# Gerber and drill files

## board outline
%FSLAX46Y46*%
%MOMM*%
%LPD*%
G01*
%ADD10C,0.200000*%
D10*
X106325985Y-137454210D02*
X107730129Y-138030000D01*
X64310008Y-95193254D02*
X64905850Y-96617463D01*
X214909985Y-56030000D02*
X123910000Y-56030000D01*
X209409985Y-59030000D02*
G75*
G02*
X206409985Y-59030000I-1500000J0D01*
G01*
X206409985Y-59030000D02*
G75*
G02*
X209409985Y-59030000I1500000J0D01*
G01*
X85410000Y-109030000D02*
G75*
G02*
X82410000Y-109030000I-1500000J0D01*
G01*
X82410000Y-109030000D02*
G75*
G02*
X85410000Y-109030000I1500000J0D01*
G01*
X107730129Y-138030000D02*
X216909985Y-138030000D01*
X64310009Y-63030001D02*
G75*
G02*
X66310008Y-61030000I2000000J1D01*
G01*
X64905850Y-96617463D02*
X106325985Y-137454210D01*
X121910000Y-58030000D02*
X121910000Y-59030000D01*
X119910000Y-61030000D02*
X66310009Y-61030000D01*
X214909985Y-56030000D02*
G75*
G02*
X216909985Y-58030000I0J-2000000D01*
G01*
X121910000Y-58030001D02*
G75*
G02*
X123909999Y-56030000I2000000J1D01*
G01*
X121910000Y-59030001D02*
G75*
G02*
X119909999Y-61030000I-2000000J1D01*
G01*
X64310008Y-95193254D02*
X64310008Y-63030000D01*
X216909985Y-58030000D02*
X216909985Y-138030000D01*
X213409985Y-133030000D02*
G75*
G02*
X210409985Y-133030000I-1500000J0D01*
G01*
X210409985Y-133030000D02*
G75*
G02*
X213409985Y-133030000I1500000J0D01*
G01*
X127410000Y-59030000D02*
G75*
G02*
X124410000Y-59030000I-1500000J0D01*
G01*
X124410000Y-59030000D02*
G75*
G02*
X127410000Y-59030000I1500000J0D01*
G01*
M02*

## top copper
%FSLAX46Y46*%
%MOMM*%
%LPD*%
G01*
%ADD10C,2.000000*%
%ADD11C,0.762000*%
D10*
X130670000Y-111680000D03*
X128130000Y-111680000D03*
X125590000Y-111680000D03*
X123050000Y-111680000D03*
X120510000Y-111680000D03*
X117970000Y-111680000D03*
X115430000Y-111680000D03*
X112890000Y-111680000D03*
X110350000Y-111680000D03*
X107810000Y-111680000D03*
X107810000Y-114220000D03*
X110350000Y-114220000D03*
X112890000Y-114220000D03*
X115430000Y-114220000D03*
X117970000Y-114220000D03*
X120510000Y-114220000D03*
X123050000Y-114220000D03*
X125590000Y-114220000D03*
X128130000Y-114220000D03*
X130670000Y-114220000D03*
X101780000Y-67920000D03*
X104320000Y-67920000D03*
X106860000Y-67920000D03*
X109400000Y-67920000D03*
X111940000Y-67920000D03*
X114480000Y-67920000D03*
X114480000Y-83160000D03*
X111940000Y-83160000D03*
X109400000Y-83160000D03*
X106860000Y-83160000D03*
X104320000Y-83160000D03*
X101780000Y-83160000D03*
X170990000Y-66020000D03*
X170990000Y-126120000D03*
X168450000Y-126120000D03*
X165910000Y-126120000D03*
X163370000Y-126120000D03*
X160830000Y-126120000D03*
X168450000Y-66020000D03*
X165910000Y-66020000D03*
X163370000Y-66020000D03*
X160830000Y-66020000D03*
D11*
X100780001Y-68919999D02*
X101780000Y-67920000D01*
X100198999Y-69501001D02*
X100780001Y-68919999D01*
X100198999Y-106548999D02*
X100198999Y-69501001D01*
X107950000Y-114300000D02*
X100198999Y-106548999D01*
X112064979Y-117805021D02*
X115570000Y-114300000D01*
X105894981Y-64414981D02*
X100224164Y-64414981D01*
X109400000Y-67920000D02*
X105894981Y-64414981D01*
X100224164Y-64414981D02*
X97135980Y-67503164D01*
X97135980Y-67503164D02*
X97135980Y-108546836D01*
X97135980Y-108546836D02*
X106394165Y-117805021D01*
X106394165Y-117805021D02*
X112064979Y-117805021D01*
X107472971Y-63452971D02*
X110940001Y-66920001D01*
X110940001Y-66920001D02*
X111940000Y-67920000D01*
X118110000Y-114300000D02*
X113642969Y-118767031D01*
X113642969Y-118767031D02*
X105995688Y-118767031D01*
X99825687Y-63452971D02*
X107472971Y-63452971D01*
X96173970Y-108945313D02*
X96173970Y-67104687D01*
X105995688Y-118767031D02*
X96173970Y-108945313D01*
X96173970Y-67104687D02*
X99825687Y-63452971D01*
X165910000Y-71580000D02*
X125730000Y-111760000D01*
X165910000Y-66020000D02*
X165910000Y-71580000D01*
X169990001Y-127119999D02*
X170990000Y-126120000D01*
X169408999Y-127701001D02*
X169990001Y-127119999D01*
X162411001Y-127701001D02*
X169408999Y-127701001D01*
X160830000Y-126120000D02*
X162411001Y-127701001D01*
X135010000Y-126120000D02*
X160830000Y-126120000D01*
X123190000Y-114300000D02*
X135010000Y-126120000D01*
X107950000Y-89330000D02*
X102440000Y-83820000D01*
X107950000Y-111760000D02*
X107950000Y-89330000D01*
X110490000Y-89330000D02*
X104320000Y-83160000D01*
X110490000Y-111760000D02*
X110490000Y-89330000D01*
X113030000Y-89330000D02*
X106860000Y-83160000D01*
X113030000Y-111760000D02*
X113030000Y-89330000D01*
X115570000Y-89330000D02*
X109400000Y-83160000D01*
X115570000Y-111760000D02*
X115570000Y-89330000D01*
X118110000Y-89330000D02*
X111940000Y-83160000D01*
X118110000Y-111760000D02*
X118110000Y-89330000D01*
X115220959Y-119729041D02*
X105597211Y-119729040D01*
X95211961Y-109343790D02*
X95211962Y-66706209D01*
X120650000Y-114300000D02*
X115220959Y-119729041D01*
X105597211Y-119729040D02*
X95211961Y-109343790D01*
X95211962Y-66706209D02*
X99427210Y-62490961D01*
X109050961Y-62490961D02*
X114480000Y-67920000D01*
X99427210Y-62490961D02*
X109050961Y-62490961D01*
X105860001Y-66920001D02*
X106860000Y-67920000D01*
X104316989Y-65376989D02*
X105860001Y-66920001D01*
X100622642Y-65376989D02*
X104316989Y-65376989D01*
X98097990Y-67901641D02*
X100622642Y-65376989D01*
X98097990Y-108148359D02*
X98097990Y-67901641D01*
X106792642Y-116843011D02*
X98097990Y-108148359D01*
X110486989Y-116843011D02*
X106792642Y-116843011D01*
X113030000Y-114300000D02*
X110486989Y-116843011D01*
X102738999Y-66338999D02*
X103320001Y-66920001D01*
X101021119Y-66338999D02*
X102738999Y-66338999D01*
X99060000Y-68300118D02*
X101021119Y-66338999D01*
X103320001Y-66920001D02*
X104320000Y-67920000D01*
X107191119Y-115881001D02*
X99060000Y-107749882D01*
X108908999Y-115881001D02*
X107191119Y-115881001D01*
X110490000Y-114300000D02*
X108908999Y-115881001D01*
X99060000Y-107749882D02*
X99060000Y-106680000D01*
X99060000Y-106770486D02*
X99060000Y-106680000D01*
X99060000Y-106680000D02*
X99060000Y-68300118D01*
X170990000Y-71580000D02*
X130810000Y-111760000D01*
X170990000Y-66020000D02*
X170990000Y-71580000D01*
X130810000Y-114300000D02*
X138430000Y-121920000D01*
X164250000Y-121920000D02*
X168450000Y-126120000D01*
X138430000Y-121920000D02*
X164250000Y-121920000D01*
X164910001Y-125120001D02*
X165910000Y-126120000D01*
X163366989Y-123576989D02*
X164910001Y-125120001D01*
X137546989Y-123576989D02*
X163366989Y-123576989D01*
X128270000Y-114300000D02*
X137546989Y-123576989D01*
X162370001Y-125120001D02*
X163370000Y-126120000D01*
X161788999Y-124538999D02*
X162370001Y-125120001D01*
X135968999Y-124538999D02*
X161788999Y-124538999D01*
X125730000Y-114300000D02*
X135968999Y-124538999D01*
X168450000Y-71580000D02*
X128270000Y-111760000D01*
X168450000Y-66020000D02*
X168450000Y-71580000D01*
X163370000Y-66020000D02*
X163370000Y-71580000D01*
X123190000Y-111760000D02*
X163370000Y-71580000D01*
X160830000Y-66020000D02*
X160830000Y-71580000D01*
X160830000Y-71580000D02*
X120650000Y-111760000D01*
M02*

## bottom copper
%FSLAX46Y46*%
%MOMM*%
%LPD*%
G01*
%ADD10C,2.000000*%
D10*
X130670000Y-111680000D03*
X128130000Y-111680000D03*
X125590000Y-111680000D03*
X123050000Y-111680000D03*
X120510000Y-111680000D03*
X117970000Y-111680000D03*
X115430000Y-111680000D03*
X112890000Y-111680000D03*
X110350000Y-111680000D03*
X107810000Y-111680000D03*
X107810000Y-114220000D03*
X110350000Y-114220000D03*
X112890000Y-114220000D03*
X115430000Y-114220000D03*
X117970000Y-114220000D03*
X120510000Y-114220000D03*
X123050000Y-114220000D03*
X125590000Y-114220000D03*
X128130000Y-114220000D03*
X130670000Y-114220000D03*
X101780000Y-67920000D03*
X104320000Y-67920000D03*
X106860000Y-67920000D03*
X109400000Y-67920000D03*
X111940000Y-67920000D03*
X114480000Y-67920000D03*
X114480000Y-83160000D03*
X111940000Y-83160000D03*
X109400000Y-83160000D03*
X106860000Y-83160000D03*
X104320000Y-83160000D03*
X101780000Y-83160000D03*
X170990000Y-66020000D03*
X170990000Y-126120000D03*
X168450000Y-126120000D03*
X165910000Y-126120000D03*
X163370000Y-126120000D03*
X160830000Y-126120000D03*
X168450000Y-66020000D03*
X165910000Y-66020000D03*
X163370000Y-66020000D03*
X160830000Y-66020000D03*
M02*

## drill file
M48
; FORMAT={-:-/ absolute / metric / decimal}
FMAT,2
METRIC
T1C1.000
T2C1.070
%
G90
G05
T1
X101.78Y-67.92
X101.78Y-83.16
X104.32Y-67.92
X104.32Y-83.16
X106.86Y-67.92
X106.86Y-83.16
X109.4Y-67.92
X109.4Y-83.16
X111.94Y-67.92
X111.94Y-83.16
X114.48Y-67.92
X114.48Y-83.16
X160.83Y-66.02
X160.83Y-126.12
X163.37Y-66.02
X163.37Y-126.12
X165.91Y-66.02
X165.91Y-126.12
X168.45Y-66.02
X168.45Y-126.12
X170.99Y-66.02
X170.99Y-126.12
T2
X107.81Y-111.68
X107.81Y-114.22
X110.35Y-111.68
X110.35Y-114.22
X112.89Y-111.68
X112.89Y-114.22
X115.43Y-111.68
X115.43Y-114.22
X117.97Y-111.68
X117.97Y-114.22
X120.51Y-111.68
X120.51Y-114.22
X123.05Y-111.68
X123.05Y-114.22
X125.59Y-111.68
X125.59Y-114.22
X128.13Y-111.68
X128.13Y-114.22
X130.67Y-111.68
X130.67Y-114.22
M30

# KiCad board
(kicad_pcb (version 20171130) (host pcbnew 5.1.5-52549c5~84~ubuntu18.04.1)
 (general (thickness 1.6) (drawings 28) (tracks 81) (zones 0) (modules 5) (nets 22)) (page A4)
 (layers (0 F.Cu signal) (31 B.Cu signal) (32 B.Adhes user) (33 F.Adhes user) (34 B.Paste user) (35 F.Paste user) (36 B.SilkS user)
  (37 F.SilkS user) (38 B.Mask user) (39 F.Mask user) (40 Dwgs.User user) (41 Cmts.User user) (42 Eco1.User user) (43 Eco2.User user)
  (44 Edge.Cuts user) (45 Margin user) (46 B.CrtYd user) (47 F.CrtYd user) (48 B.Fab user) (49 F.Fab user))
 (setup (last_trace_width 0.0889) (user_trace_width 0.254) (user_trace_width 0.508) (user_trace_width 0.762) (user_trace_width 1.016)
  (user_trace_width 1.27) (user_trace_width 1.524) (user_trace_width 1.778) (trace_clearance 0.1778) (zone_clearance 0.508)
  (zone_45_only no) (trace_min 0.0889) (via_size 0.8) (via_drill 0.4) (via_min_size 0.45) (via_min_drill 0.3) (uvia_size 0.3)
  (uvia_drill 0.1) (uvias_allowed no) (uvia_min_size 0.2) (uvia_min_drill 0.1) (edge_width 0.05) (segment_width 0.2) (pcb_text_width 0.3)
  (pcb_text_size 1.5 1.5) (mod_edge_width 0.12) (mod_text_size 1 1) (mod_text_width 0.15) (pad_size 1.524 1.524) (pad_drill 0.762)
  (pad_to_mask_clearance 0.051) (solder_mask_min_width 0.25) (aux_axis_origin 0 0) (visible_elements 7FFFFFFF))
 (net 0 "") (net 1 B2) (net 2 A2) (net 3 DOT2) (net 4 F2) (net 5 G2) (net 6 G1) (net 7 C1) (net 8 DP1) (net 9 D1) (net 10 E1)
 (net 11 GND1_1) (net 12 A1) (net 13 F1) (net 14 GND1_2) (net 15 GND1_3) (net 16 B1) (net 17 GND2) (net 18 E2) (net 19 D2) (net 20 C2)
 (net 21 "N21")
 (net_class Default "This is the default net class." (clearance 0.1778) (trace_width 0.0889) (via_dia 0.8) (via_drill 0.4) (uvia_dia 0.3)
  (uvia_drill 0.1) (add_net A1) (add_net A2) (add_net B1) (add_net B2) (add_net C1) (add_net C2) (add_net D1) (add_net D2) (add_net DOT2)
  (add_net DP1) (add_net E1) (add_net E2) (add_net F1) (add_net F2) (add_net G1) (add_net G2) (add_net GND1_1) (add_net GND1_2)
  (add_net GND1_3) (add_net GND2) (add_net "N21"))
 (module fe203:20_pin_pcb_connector (layer B.Cu) (at 161.29 114.22 180)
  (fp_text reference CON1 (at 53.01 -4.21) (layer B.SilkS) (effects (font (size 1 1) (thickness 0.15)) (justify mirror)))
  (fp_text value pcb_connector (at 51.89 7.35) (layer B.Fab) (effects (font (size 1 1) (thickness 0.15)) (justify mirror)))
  (pad 2 thru_hole circle (at 30.62 2.54 180) (size 2 2) (drill 1.07) (layers *.Cu *.Mask) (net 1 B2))
  (pad 4 thru_hole circle (at 33.16 2.54 180) (size 2 2) (drill 1.07) (layers *.Cu *.Mask) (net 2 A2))
  (pad 6 thru_hole circle (at 35.7 2.54 180) (size 2 2) (drill 1.07) (layers *.Cu *.Mask) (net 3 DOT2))
  (pad 8 thru_hole circle (at 38.24 2.54 180) (size 2 2) (drill 1.07) (layers *.Cu *.Mask) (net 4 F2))
  (pad 10 thru_hole circle (at 40.78 2.54 180) (size 2 2) (drill 1.07) (layers *.Cu *.Mask) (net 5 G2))
  (pad 12 thru_hole circle (at 43.32 2.54 180) (size 2 2) (drill 1.07) (layers *.Cu *.Mask) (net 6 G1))
  (pad 14 thru_hole circle (at 45.86 2.54 180) (size 2 2) (drill 1.07) (layers *.Cu *.Mask) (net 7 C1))
  (pad 16 thru_hole circle (at 48.4 2.54 180) (size 2 2) (drill 1.07) (layers *.Cu *.Mask) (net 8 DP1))
  (pad 18 thru_hole circle (at 50.94 2.54 180) (size 2 2) (drill 1.07) (layers *.Cu *.Mask) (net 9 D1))
  (pad 20 thru_hole circle (at 53.48 2.54 180) (size 2 2) (drill 1.07) (layers *.Cu *.Mask) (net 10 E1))
  (pad 19 thru_hole circle (at 53.48 0 180) (size 2 2) (drill 1.07) (layers *.Cu *.Mask) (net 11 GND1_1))
  (pad 17 thru_hole circle (at 50.94 0 180) (size 2 2) (drill 1.07) (layers *.Cu *.Mask) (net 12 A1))
  (pad 15 thru_hole circle (at 48.4 0 180) (size 2 2) (drill 1.07) (layers *.Cu *.Mask) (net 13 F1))
  (pad 13 thru_hole circle (at 45.86 0 180) (size 2 2) (drill 1.07) (layers *.Cu *.Mask) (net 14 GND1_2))
  (pad 11 thru_hole circle (at 43.32 0 180) (size 2 2) (drill 1.07) (layers *.Cu *.Mask) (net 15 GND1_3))
  (pad 9 thru_hole circle (at 40.78 0 180) (size 2 2) (drill 1.07) (layers *.Cu *.Mask) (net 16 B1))
  (pad 7 thru_hole circle (at 38.24 0 180) (size 2 2) (drill 1.07) (layers *.Cu *.Mask) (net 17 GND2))
  (pad 5 thru_hole circle (at 35.7 0 180) (size 2 2) (drill 1.07) (layers *.Cu *.Mask) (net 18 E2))
  (pad 3 thru_hole circle (at 33.16 0 180) (size 2 2) (drill 1.07) (layers *.Cu *.Mask) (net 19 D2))
  (pad 1 thru_hole circle (at 30.62 0 180) (size 2 2) (drill 1.07) (layers *.Cu *.Mask) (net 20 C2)))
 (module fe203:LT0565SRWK (layer F.Cu) (at 89.08 85.7)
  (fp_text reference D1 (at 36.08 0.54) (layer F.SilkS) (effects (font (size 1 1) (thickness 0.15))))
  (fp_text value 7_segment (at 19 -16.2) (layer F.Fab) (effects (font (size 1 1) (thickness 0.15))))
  (pad 12 thru_hole circle (at 12.7 -17.78) (size 2 2) (drill 1) (layers *.Cu *.Mask) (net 11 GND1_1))
  (pad 11 thru_hole circle (at 15.24 -17.78) (size 2 2) (drill 1) (layers *.Cu *.Mask) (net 12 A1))
  (pad 10 thru_hole circle (at 17.78 -17.78) (size 2 2) (drill 1) (layers *.Cu *.Mask) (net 13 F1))
  (pad 9 thru_hole circle (at 20.32 -17.78) (size 2 2) (drill 1) (layers *.Cu *.Mask) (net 14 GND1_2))
  (pad 8 thru_hole circle (at 22.86 -17.78) (size 2 2) (drill 1) (layers *.Cu *.Mask) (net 15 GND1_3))
  (pad 7 thru_hole circle (at 25.4 -17.78) (size 2 2) (drill 1) (layers *.Cu *.Mask) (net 16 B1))
  (pad 6 thru_hole circle (at 25.4 -2.54) (size 2 2) (drill 1) (layers *.Cu *.Mask) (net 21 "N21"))
  (pad 5 thru_hole circle (at 22.86 -2.54) (size 2 2) (drill 1) (layers *.Cu *.Mask) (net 6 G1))
  (pad 4 thru_hole circle (at 20.32 -2.54) (size 2 2) (drill 1) (layers *.Cu *.Mask) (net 7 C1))
  (pad 3 thru_hole circle (at 17.78 -2.54) (size 2 2) (drill 1) (layers *.Cu *.Mask) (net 8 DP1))
  (pad 2 thru_hole circle (at 15.24 -2.54) (size 2 2) (drill 1) (layers *.Cu *.Mask) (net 9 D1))
  (pad 1 thru_hole circle (at 12.7 -2.54) (size 2 2) (drill 1) (layers *.Cu *.Mask) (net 10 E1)))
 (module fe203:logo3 (layer F.Cu) (at 161.23 99.49)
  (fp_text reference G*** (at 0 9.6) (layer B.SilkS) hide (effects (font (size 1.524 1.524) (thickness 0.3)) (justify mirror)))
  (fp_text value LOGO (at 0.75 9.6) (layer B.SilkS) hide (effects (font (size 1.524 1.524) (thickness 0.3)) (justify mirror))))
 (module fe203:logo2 (layer F.Cu) (at 174.63 93.98)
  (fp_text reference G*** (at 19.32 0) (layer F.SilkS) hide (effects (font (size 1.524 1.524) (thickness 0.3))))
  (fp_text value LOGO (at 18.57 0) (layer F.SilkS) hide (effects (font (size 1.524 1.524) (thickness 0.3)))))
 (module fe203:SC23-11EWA (layer F.Cu) (at 165.91 126.12)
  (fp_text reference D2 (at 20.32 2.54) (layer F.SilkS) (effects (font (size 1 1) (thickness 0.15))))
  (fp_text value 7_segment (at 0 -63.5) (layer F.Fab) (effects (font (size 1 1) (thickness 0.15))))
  (pad 6 thru_hole circle (at 5.08 -60.1) (size 2 2) (drill 1) (layers *.Cu *.Mask) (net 1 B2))
  (pad 5 thru_hole circle (at 5.08 0) (size 2 2) (drill 1) (layers *.Cu *.Mask) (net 17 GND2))
  (pad 4 thru_hole circle (at 2.54 0) (size 2 2) (drill 1) (layers *.Cu *.Mask) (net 20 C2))
  (pad 3 thru_hole circle (at 0 0) (size 2 2) (drill 1) (layers *.Cu *.Mask) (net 19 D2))
  (pad 2 thru_hole circle (at -2.54 0) (size 2 2) (drill 1) (layers *.Cu *.Mask) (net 18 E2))
  (pad 1 thru_hole circle (at -5.08 0) (size 2 2) (drill 1) (layers *.Cu *.Mask) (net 17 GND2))
  (pad 7 thru_hole circle (at 2.54 -60.1) (size 2 2) (drill 1) (layers *.Cu *.Mask) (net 2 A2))
  (pad 8 thru_hole circle (at 0 -60.1) (size 2 2) (drill 1) (layers *.Cu *.Mask) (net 3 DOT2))
  (pad 9 thru_hole circle (at -2.54 -60.1) (size 2 2) (drill 1) (layers *.Cu *.Mask) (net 4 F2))
  (pad 10 thru_hole circle (at -5.08 -60.1) (size 2 2) (drill 1) (layers *.Cu *.Mask) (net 5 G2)))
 (gr_line (start 106.325985 137.45421) (end 107.730129 138.03) (layer Edge.Cuts) (width 0.2))
 (gr_line (start 64.310008 95.193254) (end 64.90585 96.617463) (layer Edge.Cuts) (width 0.2))
 (gr_line (start 214.909985 56.03) (end 123.91 56.03) (layer Edge.Cuts) (width 0.2))
 (gr_circle (center 207.909985 59.03) (end 209.409985 59.03) (layer Edge.Cuts) (width 0.2))
 (gr_circle (center 83.91 109.03) (end 85.41 109.03) (layer Edge.Cuts) (width 0.2))
 (gr_line (start 107.730129 138.03) (end 216.909985 138.03) (layer Edge.Cuts) (width 0.2))
 (gr_arc (start 66.310009 63.03) (end 66.310008 61.03) (angle -90) (layer Edge.Cuts) (width 0.2))
 (gr_line (start 64.90585 96.617463) (end 106.325985 137.45421) (layer Edge.Cuts) (width 0.2))
 (gr_line (start 121.91 58.03) (end 121.91 59.03) (layer Edge.Cuts) (width 0.2))
 (gr_line (start 119.91 61.03) (end 66.310009 61.03) (layer Edge.Cuts) (width 0.2))
 (gr_arc (start 214.909985 58.03) (end 216.909985 58.03) (angle -90) (layer Edge.Cuts) (width 0.2))
 (gr_arc (start 123.91 58.03) (end 123.909999 56.03) (angle -90) (layer Edge.Cuts) (width 0.2))
 (gr_arc (start 119.91 59.03) (end 119.909999 61.03) (angle -90) (layer Edge.Cuts) (width 0.2))
 (gr_line (start 64.310008 95.193254) (end 64.310008 63.03) (layer Edge.Cuts) (width 0.2))
 (gr_line (start 216.909985 58.03) (end 216.909985 138.03) (layer Edge.Cuts) (width 0.2))
 (gr_circle (center 211.909985 133.03) (end 213.409985 133.03) (layer Edge.Cuts) (width 0.2))
 (gr_circle (center 125.91 59.03) (end 127.41 59.03) (layer Edge.Cuts) (width 0.2))
 (segment (start 100.780001 68.919999) (end 101.78 67.92) (width 0.762) (layer F.Cu) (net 11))
 (segment (start 100.198999 69.501001) (end 100.780001 68.919999) (width 0.762) (layer F.Cu) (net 11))
 (segment (start 100.198999 106.548999) (end 100.198999 69.501001) (width 0.762) (layer F.Cu) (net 11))
 (segment (start 107.95 114.3) (end 100.198999 106.548999) (width 0.762) (layer F.Cu) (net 11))
 (segment (start 112.064979 117.805021) (end 115.57 114.3) (width 0.762) (layer F.Cu) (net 14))
 (segment (start 105.894981 64.414981) (end 100.224164 64.414981) (width 0.762) (layer F.Cu) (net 14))
 (segment (start 109.4 67.92) (end 105.894981 64.414981) (width 0.762) (layer F.Cu) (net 14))
 (segment (start 100.224164 64.414981) (end 97.13598 67.503164) (width 0.762) (layer F.Cu) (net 14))
 (segment (start 97.13598 67.503164) (end 97.13598 108.546836) (width 0.762) (layer F.Cu) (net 14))
 (segment (start 97.13598 108.546836) (end 106.394165 117.805021) (width 0.762) (layer F.Cu) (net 14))
 (segment (start 106.394165 117.805021) (end 112.064979 117.805021) (width 0.762) (layer F.Cu) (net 14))
 (segment (start 107.472971 63.452971) (end 110.940001 66.920001) (width 0.762) (layer F.Cu) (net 15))
 (segment (start 110.940001 66.920001) (end 111.94 67.92) (width 0.762) (layer F.Cu) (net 15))
 (segment (start 118.11 114.3) (end 113.642969 118.767031) (width 0.762) (layer F.Cu) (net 15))
 (segment (start 113.642969 118.767031) (end 105.995688 118.767031) (width 0.762) (layer F.Cu) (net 15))
 (segment (start 99.825687 63.452971) (end 107.472971 63.452971) (width 0.762) (layer F.Cu) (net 15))
 (segment (start 96.17397 108.945313) (end 96.17397 67.104687) (width 0.762) (layer F.Cu) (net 15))
 (segment (start 105.995688 118.767031) (end 96.17397 108.945313) (width 0.762) (layer F.Cu) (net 15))
 (segment (start 96.17397 67.104687) (end 99.825687 63.452971) (width 0.762) (layer F.Cu) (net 15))
 (segment (start 165.91 71.58) (end 125.73 111.76) (width 0.762) (layer F.Cu) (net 3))
 (segment (start 165.91 66.02) (end 165.91 71.58) (width 0.762) (layer F.Cu) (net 3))
 (segment (start 169.990001 127.119999) (end 170.99 126.12) (width 0.762) (layer F.Cu) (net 17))
 (segment (start 169.408999 127.701001) (end 169.990001 127.119999) (width 0.762) (layer F.Cu) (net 17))
 (segment (start 162.411001 127.701001) (end 169.408999 127.701001) (width 0.762) (layer F.Cu) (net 17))
 (segment (start 160.83 126.12) (end 162.411001 127.701001) (width 0.762) (layer F.Cu) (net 17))
 (segment (start 135.01 126.12) (end 160.83 126.12) (width 0.762) (layer F.Cu) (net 17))
 (segment (start 123.19 114.3) (end 135.01 126.12) (width 0.762) (layer F.Cu) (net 17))
 (segment (start 107.95 89.33) (end 102.44 83.82) (width 0.762) (layer F.Cu) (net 10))
 (segment (start 107.95 111.76) (end 107.95 89.33) (width 0.762) (layer F.Cu) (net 10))
 (segment (start 110.49 89.33) (end 104.32 83.16) (width 0.762) (layer F.Cu) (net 9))
 (segment (start 110.49 111.76) (end 110.49 89.33) (width 0.762) (layer F.Cu) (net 9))
 (segment (start 113.03 89.33) (end 106.86 83.16) (width 0.762) (layer F.Cu) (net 8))
 (segment (start 113.03 111.76) (end 113.03 89.33) (width 0.762) (layer F.Cu) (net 8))
 (segment (start 115.57 89.33) (end 109.4 83.16) (width 0.762) (layer F.Cu) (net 7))
 (segment (start 115.57 111.76) (end 115.57 89.33) (width 0.762) (layer F.Cu) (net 7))
 (segment (start 118.11 89.33) (end 111.94 83.16) (width 0.762) (layer F.Cu) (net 6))
 (segment (start 118.11 111.76) (end 118.11 89.33) (width 0.762) (layer F.Cu) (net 6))
 (segment (start 115.220959 119.729041) (end 105.597211 119.72904) (width 0.762) (layer F.Cu) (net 16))
 (segment (start 95.211961 109.34379) (end 95.211962 66.706209) (width 0.762) (layer F.Cu) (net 16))
 (segment (start 120.65 114.3) (end 115.220959 119.729041) (width 0.762) (layer F.Cu) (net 16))
 (segment (start 105.597211 119.72904) (end 95.211961 109.34379) (width 0.762) (layer F.Cu) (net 16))
 (segment (start 95.211962 66.706209) (end 99.42721 62.490961) (width 0.762) (layer F.Cu) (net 16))
 (segment (start 109.050961 62.490961) (end 114.48 67.92) (width 0.762) (layer F.Cu) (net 16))
 (segment (start 99.42721 62.490961) (end 109.050961 62.490961) (width 0.762) (layer F.Cu) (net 16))
 (segment (start 105.860001 66.920001) (end 106.86 67.92) (width 0.762) (layer F.Cu) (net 13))
 (segment (start 104.316989 65.376989) (end 105.860001 66.920001) (width 0.762) (layer F.Cu) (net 13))
 (segment (start 100.622642 65.376989) (end 104.316989 65.376989) (width 0.762) (layer F.Cu) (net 13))
 (segment (start 98.09799 67.901641) (end 100.622642 65.376989) (width 0.762) (layer F.Cu) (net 13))
 (segment (start 98.09799 108.148359) (end 98.09799 67.901641) (width 0.762) (layer F.Cu) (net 13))
 (segment (start 106.792642 116.843011) (end 98.09799 108.148359) (width 0.762) (layer F.Cu) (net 13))
 (segment (start 110.486989 116.843011) (end 106.792642 116.843011) (width 0.762) (layer F.Cu) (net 13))
 (segment (start 113.03 114.3) (end 110.486989 116.843011) (width 0.762) (layer F.Cu) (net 13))
 (segment (start 102.738999 66.338999) (end 103.320001 66.920001) (width 0.762) (layer F.Cu) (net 12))
 (segment (start 101.021119 66.338999) (end 102.738999 66.338999) (width 0.762) (layer F.Cu) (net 12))
 (segment (start 99.06 68.300118) (end 101.021119 66.338999) (width 0.762) (layer F.Cu) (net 12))
 (segment (start 103.320001 66.920001) (end 104.32 67.92) (width 0.762) (layer F.Cu) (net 12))
 (segment (start 107.191119 115.881001) (end 99.06 107.749882) (width 0.762) (layer F.Cu) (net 12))
 (segment (start 108.908999 115.881001) (end 107.191119 115.881001) (width 0.762) (layer F.Cu) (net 12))
 (segment (start 110.49 114.3) (end 108.908999 115.881001) (width 0.762) (layer F.Cu) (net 12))
 (segment (start 99.06 107.749882) (end 99.06 106.68) (width 0.762) (layer F.Cu) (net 12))
 (segment (start 99.06 106.770486) (end 99.06 106.68) (width 0.762) (layer F.Cu) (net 12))
 (segment (start 99.06 106.68) (end 99.06 68.300118) (width 0.762) (layer F.Cu) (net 12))
 (segment (start 170.99 71.58) (end 130.81 111.76) (width 0.762) (layer F.Cu) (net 1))
 (segment (start 170.99 66.02) (end 170.99 71.58) (width 0.762) (layer F.Cu) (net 1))
 (segment (start 130.81 114.3) (end 138.43 121.92) (width 0.762) (layer F.Cu) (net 20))
 (segment (start 164.25 121.92) (end 168.45 126.12) (width 0.762) (layer F.Cu) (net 20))
 (segment (start 138.43 121.92) (end 164.25 121.92) (width 0.762) (layer F.Cu) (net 20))
 (segment (start 164.910001 125.120001) (end 165.91 126.12) (width 0.762) (layer F.Cu) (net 19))
 (segment (start 163.366989 123.576989) (end 164.910001 125.120001) (width 0.762) (layer F.Cu) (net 19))
 (segment (start 137.546989 123.576989) (end 163.366989 123.576989) (width 0.762) (layer F.Cu) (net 19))
 (segment (start 128.27 114.3) (end 137.546989 123.576989) (width 0.762) (layer F.Cu) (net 19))
 (segment (start 162.370001 125.120001) (end 163.37 126.12) (width 0.762) (layer F.Cu) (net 18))
 (segment (start 161.788999 124.538999) (end 162.370001 125.120001) (width 0.762) (layer F.Cu) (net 18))
 (segment (start 135.968999 124.538999) (end 161.788999 124.538999) (width 0.762) (layer F.Cu) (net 18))
 (segment (start 125.73 114.3) (end 135.968999 124.538999) (width 0.762) (layer F.Cu) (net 18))
 (segment (start 168.45 71.58) (end 128.27 111.76) (width 0.762) (layer F.Cu) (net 2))
 (segment (start 168.45 66.02) (end 168.45 71.58) (width 0.762) (layer F.Cu) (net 2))
 (segment (start 163.37 66.02) (end 163.37 71.58) (width 0.762) (layer F.Cu) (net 4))
 (segment (start 123.19 111.76) (end 163.37 71.58) (width 0.762) (layer F.Cu) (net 4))
 (segment (start 160.83 66.02) (end 160.83 71.58) (width 0.762) (layer F.Cu) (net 5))
 (segment (start 160.83 71.58) (end 120.65 111.76) (width 0.762) (layer F.Cu) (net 5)))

